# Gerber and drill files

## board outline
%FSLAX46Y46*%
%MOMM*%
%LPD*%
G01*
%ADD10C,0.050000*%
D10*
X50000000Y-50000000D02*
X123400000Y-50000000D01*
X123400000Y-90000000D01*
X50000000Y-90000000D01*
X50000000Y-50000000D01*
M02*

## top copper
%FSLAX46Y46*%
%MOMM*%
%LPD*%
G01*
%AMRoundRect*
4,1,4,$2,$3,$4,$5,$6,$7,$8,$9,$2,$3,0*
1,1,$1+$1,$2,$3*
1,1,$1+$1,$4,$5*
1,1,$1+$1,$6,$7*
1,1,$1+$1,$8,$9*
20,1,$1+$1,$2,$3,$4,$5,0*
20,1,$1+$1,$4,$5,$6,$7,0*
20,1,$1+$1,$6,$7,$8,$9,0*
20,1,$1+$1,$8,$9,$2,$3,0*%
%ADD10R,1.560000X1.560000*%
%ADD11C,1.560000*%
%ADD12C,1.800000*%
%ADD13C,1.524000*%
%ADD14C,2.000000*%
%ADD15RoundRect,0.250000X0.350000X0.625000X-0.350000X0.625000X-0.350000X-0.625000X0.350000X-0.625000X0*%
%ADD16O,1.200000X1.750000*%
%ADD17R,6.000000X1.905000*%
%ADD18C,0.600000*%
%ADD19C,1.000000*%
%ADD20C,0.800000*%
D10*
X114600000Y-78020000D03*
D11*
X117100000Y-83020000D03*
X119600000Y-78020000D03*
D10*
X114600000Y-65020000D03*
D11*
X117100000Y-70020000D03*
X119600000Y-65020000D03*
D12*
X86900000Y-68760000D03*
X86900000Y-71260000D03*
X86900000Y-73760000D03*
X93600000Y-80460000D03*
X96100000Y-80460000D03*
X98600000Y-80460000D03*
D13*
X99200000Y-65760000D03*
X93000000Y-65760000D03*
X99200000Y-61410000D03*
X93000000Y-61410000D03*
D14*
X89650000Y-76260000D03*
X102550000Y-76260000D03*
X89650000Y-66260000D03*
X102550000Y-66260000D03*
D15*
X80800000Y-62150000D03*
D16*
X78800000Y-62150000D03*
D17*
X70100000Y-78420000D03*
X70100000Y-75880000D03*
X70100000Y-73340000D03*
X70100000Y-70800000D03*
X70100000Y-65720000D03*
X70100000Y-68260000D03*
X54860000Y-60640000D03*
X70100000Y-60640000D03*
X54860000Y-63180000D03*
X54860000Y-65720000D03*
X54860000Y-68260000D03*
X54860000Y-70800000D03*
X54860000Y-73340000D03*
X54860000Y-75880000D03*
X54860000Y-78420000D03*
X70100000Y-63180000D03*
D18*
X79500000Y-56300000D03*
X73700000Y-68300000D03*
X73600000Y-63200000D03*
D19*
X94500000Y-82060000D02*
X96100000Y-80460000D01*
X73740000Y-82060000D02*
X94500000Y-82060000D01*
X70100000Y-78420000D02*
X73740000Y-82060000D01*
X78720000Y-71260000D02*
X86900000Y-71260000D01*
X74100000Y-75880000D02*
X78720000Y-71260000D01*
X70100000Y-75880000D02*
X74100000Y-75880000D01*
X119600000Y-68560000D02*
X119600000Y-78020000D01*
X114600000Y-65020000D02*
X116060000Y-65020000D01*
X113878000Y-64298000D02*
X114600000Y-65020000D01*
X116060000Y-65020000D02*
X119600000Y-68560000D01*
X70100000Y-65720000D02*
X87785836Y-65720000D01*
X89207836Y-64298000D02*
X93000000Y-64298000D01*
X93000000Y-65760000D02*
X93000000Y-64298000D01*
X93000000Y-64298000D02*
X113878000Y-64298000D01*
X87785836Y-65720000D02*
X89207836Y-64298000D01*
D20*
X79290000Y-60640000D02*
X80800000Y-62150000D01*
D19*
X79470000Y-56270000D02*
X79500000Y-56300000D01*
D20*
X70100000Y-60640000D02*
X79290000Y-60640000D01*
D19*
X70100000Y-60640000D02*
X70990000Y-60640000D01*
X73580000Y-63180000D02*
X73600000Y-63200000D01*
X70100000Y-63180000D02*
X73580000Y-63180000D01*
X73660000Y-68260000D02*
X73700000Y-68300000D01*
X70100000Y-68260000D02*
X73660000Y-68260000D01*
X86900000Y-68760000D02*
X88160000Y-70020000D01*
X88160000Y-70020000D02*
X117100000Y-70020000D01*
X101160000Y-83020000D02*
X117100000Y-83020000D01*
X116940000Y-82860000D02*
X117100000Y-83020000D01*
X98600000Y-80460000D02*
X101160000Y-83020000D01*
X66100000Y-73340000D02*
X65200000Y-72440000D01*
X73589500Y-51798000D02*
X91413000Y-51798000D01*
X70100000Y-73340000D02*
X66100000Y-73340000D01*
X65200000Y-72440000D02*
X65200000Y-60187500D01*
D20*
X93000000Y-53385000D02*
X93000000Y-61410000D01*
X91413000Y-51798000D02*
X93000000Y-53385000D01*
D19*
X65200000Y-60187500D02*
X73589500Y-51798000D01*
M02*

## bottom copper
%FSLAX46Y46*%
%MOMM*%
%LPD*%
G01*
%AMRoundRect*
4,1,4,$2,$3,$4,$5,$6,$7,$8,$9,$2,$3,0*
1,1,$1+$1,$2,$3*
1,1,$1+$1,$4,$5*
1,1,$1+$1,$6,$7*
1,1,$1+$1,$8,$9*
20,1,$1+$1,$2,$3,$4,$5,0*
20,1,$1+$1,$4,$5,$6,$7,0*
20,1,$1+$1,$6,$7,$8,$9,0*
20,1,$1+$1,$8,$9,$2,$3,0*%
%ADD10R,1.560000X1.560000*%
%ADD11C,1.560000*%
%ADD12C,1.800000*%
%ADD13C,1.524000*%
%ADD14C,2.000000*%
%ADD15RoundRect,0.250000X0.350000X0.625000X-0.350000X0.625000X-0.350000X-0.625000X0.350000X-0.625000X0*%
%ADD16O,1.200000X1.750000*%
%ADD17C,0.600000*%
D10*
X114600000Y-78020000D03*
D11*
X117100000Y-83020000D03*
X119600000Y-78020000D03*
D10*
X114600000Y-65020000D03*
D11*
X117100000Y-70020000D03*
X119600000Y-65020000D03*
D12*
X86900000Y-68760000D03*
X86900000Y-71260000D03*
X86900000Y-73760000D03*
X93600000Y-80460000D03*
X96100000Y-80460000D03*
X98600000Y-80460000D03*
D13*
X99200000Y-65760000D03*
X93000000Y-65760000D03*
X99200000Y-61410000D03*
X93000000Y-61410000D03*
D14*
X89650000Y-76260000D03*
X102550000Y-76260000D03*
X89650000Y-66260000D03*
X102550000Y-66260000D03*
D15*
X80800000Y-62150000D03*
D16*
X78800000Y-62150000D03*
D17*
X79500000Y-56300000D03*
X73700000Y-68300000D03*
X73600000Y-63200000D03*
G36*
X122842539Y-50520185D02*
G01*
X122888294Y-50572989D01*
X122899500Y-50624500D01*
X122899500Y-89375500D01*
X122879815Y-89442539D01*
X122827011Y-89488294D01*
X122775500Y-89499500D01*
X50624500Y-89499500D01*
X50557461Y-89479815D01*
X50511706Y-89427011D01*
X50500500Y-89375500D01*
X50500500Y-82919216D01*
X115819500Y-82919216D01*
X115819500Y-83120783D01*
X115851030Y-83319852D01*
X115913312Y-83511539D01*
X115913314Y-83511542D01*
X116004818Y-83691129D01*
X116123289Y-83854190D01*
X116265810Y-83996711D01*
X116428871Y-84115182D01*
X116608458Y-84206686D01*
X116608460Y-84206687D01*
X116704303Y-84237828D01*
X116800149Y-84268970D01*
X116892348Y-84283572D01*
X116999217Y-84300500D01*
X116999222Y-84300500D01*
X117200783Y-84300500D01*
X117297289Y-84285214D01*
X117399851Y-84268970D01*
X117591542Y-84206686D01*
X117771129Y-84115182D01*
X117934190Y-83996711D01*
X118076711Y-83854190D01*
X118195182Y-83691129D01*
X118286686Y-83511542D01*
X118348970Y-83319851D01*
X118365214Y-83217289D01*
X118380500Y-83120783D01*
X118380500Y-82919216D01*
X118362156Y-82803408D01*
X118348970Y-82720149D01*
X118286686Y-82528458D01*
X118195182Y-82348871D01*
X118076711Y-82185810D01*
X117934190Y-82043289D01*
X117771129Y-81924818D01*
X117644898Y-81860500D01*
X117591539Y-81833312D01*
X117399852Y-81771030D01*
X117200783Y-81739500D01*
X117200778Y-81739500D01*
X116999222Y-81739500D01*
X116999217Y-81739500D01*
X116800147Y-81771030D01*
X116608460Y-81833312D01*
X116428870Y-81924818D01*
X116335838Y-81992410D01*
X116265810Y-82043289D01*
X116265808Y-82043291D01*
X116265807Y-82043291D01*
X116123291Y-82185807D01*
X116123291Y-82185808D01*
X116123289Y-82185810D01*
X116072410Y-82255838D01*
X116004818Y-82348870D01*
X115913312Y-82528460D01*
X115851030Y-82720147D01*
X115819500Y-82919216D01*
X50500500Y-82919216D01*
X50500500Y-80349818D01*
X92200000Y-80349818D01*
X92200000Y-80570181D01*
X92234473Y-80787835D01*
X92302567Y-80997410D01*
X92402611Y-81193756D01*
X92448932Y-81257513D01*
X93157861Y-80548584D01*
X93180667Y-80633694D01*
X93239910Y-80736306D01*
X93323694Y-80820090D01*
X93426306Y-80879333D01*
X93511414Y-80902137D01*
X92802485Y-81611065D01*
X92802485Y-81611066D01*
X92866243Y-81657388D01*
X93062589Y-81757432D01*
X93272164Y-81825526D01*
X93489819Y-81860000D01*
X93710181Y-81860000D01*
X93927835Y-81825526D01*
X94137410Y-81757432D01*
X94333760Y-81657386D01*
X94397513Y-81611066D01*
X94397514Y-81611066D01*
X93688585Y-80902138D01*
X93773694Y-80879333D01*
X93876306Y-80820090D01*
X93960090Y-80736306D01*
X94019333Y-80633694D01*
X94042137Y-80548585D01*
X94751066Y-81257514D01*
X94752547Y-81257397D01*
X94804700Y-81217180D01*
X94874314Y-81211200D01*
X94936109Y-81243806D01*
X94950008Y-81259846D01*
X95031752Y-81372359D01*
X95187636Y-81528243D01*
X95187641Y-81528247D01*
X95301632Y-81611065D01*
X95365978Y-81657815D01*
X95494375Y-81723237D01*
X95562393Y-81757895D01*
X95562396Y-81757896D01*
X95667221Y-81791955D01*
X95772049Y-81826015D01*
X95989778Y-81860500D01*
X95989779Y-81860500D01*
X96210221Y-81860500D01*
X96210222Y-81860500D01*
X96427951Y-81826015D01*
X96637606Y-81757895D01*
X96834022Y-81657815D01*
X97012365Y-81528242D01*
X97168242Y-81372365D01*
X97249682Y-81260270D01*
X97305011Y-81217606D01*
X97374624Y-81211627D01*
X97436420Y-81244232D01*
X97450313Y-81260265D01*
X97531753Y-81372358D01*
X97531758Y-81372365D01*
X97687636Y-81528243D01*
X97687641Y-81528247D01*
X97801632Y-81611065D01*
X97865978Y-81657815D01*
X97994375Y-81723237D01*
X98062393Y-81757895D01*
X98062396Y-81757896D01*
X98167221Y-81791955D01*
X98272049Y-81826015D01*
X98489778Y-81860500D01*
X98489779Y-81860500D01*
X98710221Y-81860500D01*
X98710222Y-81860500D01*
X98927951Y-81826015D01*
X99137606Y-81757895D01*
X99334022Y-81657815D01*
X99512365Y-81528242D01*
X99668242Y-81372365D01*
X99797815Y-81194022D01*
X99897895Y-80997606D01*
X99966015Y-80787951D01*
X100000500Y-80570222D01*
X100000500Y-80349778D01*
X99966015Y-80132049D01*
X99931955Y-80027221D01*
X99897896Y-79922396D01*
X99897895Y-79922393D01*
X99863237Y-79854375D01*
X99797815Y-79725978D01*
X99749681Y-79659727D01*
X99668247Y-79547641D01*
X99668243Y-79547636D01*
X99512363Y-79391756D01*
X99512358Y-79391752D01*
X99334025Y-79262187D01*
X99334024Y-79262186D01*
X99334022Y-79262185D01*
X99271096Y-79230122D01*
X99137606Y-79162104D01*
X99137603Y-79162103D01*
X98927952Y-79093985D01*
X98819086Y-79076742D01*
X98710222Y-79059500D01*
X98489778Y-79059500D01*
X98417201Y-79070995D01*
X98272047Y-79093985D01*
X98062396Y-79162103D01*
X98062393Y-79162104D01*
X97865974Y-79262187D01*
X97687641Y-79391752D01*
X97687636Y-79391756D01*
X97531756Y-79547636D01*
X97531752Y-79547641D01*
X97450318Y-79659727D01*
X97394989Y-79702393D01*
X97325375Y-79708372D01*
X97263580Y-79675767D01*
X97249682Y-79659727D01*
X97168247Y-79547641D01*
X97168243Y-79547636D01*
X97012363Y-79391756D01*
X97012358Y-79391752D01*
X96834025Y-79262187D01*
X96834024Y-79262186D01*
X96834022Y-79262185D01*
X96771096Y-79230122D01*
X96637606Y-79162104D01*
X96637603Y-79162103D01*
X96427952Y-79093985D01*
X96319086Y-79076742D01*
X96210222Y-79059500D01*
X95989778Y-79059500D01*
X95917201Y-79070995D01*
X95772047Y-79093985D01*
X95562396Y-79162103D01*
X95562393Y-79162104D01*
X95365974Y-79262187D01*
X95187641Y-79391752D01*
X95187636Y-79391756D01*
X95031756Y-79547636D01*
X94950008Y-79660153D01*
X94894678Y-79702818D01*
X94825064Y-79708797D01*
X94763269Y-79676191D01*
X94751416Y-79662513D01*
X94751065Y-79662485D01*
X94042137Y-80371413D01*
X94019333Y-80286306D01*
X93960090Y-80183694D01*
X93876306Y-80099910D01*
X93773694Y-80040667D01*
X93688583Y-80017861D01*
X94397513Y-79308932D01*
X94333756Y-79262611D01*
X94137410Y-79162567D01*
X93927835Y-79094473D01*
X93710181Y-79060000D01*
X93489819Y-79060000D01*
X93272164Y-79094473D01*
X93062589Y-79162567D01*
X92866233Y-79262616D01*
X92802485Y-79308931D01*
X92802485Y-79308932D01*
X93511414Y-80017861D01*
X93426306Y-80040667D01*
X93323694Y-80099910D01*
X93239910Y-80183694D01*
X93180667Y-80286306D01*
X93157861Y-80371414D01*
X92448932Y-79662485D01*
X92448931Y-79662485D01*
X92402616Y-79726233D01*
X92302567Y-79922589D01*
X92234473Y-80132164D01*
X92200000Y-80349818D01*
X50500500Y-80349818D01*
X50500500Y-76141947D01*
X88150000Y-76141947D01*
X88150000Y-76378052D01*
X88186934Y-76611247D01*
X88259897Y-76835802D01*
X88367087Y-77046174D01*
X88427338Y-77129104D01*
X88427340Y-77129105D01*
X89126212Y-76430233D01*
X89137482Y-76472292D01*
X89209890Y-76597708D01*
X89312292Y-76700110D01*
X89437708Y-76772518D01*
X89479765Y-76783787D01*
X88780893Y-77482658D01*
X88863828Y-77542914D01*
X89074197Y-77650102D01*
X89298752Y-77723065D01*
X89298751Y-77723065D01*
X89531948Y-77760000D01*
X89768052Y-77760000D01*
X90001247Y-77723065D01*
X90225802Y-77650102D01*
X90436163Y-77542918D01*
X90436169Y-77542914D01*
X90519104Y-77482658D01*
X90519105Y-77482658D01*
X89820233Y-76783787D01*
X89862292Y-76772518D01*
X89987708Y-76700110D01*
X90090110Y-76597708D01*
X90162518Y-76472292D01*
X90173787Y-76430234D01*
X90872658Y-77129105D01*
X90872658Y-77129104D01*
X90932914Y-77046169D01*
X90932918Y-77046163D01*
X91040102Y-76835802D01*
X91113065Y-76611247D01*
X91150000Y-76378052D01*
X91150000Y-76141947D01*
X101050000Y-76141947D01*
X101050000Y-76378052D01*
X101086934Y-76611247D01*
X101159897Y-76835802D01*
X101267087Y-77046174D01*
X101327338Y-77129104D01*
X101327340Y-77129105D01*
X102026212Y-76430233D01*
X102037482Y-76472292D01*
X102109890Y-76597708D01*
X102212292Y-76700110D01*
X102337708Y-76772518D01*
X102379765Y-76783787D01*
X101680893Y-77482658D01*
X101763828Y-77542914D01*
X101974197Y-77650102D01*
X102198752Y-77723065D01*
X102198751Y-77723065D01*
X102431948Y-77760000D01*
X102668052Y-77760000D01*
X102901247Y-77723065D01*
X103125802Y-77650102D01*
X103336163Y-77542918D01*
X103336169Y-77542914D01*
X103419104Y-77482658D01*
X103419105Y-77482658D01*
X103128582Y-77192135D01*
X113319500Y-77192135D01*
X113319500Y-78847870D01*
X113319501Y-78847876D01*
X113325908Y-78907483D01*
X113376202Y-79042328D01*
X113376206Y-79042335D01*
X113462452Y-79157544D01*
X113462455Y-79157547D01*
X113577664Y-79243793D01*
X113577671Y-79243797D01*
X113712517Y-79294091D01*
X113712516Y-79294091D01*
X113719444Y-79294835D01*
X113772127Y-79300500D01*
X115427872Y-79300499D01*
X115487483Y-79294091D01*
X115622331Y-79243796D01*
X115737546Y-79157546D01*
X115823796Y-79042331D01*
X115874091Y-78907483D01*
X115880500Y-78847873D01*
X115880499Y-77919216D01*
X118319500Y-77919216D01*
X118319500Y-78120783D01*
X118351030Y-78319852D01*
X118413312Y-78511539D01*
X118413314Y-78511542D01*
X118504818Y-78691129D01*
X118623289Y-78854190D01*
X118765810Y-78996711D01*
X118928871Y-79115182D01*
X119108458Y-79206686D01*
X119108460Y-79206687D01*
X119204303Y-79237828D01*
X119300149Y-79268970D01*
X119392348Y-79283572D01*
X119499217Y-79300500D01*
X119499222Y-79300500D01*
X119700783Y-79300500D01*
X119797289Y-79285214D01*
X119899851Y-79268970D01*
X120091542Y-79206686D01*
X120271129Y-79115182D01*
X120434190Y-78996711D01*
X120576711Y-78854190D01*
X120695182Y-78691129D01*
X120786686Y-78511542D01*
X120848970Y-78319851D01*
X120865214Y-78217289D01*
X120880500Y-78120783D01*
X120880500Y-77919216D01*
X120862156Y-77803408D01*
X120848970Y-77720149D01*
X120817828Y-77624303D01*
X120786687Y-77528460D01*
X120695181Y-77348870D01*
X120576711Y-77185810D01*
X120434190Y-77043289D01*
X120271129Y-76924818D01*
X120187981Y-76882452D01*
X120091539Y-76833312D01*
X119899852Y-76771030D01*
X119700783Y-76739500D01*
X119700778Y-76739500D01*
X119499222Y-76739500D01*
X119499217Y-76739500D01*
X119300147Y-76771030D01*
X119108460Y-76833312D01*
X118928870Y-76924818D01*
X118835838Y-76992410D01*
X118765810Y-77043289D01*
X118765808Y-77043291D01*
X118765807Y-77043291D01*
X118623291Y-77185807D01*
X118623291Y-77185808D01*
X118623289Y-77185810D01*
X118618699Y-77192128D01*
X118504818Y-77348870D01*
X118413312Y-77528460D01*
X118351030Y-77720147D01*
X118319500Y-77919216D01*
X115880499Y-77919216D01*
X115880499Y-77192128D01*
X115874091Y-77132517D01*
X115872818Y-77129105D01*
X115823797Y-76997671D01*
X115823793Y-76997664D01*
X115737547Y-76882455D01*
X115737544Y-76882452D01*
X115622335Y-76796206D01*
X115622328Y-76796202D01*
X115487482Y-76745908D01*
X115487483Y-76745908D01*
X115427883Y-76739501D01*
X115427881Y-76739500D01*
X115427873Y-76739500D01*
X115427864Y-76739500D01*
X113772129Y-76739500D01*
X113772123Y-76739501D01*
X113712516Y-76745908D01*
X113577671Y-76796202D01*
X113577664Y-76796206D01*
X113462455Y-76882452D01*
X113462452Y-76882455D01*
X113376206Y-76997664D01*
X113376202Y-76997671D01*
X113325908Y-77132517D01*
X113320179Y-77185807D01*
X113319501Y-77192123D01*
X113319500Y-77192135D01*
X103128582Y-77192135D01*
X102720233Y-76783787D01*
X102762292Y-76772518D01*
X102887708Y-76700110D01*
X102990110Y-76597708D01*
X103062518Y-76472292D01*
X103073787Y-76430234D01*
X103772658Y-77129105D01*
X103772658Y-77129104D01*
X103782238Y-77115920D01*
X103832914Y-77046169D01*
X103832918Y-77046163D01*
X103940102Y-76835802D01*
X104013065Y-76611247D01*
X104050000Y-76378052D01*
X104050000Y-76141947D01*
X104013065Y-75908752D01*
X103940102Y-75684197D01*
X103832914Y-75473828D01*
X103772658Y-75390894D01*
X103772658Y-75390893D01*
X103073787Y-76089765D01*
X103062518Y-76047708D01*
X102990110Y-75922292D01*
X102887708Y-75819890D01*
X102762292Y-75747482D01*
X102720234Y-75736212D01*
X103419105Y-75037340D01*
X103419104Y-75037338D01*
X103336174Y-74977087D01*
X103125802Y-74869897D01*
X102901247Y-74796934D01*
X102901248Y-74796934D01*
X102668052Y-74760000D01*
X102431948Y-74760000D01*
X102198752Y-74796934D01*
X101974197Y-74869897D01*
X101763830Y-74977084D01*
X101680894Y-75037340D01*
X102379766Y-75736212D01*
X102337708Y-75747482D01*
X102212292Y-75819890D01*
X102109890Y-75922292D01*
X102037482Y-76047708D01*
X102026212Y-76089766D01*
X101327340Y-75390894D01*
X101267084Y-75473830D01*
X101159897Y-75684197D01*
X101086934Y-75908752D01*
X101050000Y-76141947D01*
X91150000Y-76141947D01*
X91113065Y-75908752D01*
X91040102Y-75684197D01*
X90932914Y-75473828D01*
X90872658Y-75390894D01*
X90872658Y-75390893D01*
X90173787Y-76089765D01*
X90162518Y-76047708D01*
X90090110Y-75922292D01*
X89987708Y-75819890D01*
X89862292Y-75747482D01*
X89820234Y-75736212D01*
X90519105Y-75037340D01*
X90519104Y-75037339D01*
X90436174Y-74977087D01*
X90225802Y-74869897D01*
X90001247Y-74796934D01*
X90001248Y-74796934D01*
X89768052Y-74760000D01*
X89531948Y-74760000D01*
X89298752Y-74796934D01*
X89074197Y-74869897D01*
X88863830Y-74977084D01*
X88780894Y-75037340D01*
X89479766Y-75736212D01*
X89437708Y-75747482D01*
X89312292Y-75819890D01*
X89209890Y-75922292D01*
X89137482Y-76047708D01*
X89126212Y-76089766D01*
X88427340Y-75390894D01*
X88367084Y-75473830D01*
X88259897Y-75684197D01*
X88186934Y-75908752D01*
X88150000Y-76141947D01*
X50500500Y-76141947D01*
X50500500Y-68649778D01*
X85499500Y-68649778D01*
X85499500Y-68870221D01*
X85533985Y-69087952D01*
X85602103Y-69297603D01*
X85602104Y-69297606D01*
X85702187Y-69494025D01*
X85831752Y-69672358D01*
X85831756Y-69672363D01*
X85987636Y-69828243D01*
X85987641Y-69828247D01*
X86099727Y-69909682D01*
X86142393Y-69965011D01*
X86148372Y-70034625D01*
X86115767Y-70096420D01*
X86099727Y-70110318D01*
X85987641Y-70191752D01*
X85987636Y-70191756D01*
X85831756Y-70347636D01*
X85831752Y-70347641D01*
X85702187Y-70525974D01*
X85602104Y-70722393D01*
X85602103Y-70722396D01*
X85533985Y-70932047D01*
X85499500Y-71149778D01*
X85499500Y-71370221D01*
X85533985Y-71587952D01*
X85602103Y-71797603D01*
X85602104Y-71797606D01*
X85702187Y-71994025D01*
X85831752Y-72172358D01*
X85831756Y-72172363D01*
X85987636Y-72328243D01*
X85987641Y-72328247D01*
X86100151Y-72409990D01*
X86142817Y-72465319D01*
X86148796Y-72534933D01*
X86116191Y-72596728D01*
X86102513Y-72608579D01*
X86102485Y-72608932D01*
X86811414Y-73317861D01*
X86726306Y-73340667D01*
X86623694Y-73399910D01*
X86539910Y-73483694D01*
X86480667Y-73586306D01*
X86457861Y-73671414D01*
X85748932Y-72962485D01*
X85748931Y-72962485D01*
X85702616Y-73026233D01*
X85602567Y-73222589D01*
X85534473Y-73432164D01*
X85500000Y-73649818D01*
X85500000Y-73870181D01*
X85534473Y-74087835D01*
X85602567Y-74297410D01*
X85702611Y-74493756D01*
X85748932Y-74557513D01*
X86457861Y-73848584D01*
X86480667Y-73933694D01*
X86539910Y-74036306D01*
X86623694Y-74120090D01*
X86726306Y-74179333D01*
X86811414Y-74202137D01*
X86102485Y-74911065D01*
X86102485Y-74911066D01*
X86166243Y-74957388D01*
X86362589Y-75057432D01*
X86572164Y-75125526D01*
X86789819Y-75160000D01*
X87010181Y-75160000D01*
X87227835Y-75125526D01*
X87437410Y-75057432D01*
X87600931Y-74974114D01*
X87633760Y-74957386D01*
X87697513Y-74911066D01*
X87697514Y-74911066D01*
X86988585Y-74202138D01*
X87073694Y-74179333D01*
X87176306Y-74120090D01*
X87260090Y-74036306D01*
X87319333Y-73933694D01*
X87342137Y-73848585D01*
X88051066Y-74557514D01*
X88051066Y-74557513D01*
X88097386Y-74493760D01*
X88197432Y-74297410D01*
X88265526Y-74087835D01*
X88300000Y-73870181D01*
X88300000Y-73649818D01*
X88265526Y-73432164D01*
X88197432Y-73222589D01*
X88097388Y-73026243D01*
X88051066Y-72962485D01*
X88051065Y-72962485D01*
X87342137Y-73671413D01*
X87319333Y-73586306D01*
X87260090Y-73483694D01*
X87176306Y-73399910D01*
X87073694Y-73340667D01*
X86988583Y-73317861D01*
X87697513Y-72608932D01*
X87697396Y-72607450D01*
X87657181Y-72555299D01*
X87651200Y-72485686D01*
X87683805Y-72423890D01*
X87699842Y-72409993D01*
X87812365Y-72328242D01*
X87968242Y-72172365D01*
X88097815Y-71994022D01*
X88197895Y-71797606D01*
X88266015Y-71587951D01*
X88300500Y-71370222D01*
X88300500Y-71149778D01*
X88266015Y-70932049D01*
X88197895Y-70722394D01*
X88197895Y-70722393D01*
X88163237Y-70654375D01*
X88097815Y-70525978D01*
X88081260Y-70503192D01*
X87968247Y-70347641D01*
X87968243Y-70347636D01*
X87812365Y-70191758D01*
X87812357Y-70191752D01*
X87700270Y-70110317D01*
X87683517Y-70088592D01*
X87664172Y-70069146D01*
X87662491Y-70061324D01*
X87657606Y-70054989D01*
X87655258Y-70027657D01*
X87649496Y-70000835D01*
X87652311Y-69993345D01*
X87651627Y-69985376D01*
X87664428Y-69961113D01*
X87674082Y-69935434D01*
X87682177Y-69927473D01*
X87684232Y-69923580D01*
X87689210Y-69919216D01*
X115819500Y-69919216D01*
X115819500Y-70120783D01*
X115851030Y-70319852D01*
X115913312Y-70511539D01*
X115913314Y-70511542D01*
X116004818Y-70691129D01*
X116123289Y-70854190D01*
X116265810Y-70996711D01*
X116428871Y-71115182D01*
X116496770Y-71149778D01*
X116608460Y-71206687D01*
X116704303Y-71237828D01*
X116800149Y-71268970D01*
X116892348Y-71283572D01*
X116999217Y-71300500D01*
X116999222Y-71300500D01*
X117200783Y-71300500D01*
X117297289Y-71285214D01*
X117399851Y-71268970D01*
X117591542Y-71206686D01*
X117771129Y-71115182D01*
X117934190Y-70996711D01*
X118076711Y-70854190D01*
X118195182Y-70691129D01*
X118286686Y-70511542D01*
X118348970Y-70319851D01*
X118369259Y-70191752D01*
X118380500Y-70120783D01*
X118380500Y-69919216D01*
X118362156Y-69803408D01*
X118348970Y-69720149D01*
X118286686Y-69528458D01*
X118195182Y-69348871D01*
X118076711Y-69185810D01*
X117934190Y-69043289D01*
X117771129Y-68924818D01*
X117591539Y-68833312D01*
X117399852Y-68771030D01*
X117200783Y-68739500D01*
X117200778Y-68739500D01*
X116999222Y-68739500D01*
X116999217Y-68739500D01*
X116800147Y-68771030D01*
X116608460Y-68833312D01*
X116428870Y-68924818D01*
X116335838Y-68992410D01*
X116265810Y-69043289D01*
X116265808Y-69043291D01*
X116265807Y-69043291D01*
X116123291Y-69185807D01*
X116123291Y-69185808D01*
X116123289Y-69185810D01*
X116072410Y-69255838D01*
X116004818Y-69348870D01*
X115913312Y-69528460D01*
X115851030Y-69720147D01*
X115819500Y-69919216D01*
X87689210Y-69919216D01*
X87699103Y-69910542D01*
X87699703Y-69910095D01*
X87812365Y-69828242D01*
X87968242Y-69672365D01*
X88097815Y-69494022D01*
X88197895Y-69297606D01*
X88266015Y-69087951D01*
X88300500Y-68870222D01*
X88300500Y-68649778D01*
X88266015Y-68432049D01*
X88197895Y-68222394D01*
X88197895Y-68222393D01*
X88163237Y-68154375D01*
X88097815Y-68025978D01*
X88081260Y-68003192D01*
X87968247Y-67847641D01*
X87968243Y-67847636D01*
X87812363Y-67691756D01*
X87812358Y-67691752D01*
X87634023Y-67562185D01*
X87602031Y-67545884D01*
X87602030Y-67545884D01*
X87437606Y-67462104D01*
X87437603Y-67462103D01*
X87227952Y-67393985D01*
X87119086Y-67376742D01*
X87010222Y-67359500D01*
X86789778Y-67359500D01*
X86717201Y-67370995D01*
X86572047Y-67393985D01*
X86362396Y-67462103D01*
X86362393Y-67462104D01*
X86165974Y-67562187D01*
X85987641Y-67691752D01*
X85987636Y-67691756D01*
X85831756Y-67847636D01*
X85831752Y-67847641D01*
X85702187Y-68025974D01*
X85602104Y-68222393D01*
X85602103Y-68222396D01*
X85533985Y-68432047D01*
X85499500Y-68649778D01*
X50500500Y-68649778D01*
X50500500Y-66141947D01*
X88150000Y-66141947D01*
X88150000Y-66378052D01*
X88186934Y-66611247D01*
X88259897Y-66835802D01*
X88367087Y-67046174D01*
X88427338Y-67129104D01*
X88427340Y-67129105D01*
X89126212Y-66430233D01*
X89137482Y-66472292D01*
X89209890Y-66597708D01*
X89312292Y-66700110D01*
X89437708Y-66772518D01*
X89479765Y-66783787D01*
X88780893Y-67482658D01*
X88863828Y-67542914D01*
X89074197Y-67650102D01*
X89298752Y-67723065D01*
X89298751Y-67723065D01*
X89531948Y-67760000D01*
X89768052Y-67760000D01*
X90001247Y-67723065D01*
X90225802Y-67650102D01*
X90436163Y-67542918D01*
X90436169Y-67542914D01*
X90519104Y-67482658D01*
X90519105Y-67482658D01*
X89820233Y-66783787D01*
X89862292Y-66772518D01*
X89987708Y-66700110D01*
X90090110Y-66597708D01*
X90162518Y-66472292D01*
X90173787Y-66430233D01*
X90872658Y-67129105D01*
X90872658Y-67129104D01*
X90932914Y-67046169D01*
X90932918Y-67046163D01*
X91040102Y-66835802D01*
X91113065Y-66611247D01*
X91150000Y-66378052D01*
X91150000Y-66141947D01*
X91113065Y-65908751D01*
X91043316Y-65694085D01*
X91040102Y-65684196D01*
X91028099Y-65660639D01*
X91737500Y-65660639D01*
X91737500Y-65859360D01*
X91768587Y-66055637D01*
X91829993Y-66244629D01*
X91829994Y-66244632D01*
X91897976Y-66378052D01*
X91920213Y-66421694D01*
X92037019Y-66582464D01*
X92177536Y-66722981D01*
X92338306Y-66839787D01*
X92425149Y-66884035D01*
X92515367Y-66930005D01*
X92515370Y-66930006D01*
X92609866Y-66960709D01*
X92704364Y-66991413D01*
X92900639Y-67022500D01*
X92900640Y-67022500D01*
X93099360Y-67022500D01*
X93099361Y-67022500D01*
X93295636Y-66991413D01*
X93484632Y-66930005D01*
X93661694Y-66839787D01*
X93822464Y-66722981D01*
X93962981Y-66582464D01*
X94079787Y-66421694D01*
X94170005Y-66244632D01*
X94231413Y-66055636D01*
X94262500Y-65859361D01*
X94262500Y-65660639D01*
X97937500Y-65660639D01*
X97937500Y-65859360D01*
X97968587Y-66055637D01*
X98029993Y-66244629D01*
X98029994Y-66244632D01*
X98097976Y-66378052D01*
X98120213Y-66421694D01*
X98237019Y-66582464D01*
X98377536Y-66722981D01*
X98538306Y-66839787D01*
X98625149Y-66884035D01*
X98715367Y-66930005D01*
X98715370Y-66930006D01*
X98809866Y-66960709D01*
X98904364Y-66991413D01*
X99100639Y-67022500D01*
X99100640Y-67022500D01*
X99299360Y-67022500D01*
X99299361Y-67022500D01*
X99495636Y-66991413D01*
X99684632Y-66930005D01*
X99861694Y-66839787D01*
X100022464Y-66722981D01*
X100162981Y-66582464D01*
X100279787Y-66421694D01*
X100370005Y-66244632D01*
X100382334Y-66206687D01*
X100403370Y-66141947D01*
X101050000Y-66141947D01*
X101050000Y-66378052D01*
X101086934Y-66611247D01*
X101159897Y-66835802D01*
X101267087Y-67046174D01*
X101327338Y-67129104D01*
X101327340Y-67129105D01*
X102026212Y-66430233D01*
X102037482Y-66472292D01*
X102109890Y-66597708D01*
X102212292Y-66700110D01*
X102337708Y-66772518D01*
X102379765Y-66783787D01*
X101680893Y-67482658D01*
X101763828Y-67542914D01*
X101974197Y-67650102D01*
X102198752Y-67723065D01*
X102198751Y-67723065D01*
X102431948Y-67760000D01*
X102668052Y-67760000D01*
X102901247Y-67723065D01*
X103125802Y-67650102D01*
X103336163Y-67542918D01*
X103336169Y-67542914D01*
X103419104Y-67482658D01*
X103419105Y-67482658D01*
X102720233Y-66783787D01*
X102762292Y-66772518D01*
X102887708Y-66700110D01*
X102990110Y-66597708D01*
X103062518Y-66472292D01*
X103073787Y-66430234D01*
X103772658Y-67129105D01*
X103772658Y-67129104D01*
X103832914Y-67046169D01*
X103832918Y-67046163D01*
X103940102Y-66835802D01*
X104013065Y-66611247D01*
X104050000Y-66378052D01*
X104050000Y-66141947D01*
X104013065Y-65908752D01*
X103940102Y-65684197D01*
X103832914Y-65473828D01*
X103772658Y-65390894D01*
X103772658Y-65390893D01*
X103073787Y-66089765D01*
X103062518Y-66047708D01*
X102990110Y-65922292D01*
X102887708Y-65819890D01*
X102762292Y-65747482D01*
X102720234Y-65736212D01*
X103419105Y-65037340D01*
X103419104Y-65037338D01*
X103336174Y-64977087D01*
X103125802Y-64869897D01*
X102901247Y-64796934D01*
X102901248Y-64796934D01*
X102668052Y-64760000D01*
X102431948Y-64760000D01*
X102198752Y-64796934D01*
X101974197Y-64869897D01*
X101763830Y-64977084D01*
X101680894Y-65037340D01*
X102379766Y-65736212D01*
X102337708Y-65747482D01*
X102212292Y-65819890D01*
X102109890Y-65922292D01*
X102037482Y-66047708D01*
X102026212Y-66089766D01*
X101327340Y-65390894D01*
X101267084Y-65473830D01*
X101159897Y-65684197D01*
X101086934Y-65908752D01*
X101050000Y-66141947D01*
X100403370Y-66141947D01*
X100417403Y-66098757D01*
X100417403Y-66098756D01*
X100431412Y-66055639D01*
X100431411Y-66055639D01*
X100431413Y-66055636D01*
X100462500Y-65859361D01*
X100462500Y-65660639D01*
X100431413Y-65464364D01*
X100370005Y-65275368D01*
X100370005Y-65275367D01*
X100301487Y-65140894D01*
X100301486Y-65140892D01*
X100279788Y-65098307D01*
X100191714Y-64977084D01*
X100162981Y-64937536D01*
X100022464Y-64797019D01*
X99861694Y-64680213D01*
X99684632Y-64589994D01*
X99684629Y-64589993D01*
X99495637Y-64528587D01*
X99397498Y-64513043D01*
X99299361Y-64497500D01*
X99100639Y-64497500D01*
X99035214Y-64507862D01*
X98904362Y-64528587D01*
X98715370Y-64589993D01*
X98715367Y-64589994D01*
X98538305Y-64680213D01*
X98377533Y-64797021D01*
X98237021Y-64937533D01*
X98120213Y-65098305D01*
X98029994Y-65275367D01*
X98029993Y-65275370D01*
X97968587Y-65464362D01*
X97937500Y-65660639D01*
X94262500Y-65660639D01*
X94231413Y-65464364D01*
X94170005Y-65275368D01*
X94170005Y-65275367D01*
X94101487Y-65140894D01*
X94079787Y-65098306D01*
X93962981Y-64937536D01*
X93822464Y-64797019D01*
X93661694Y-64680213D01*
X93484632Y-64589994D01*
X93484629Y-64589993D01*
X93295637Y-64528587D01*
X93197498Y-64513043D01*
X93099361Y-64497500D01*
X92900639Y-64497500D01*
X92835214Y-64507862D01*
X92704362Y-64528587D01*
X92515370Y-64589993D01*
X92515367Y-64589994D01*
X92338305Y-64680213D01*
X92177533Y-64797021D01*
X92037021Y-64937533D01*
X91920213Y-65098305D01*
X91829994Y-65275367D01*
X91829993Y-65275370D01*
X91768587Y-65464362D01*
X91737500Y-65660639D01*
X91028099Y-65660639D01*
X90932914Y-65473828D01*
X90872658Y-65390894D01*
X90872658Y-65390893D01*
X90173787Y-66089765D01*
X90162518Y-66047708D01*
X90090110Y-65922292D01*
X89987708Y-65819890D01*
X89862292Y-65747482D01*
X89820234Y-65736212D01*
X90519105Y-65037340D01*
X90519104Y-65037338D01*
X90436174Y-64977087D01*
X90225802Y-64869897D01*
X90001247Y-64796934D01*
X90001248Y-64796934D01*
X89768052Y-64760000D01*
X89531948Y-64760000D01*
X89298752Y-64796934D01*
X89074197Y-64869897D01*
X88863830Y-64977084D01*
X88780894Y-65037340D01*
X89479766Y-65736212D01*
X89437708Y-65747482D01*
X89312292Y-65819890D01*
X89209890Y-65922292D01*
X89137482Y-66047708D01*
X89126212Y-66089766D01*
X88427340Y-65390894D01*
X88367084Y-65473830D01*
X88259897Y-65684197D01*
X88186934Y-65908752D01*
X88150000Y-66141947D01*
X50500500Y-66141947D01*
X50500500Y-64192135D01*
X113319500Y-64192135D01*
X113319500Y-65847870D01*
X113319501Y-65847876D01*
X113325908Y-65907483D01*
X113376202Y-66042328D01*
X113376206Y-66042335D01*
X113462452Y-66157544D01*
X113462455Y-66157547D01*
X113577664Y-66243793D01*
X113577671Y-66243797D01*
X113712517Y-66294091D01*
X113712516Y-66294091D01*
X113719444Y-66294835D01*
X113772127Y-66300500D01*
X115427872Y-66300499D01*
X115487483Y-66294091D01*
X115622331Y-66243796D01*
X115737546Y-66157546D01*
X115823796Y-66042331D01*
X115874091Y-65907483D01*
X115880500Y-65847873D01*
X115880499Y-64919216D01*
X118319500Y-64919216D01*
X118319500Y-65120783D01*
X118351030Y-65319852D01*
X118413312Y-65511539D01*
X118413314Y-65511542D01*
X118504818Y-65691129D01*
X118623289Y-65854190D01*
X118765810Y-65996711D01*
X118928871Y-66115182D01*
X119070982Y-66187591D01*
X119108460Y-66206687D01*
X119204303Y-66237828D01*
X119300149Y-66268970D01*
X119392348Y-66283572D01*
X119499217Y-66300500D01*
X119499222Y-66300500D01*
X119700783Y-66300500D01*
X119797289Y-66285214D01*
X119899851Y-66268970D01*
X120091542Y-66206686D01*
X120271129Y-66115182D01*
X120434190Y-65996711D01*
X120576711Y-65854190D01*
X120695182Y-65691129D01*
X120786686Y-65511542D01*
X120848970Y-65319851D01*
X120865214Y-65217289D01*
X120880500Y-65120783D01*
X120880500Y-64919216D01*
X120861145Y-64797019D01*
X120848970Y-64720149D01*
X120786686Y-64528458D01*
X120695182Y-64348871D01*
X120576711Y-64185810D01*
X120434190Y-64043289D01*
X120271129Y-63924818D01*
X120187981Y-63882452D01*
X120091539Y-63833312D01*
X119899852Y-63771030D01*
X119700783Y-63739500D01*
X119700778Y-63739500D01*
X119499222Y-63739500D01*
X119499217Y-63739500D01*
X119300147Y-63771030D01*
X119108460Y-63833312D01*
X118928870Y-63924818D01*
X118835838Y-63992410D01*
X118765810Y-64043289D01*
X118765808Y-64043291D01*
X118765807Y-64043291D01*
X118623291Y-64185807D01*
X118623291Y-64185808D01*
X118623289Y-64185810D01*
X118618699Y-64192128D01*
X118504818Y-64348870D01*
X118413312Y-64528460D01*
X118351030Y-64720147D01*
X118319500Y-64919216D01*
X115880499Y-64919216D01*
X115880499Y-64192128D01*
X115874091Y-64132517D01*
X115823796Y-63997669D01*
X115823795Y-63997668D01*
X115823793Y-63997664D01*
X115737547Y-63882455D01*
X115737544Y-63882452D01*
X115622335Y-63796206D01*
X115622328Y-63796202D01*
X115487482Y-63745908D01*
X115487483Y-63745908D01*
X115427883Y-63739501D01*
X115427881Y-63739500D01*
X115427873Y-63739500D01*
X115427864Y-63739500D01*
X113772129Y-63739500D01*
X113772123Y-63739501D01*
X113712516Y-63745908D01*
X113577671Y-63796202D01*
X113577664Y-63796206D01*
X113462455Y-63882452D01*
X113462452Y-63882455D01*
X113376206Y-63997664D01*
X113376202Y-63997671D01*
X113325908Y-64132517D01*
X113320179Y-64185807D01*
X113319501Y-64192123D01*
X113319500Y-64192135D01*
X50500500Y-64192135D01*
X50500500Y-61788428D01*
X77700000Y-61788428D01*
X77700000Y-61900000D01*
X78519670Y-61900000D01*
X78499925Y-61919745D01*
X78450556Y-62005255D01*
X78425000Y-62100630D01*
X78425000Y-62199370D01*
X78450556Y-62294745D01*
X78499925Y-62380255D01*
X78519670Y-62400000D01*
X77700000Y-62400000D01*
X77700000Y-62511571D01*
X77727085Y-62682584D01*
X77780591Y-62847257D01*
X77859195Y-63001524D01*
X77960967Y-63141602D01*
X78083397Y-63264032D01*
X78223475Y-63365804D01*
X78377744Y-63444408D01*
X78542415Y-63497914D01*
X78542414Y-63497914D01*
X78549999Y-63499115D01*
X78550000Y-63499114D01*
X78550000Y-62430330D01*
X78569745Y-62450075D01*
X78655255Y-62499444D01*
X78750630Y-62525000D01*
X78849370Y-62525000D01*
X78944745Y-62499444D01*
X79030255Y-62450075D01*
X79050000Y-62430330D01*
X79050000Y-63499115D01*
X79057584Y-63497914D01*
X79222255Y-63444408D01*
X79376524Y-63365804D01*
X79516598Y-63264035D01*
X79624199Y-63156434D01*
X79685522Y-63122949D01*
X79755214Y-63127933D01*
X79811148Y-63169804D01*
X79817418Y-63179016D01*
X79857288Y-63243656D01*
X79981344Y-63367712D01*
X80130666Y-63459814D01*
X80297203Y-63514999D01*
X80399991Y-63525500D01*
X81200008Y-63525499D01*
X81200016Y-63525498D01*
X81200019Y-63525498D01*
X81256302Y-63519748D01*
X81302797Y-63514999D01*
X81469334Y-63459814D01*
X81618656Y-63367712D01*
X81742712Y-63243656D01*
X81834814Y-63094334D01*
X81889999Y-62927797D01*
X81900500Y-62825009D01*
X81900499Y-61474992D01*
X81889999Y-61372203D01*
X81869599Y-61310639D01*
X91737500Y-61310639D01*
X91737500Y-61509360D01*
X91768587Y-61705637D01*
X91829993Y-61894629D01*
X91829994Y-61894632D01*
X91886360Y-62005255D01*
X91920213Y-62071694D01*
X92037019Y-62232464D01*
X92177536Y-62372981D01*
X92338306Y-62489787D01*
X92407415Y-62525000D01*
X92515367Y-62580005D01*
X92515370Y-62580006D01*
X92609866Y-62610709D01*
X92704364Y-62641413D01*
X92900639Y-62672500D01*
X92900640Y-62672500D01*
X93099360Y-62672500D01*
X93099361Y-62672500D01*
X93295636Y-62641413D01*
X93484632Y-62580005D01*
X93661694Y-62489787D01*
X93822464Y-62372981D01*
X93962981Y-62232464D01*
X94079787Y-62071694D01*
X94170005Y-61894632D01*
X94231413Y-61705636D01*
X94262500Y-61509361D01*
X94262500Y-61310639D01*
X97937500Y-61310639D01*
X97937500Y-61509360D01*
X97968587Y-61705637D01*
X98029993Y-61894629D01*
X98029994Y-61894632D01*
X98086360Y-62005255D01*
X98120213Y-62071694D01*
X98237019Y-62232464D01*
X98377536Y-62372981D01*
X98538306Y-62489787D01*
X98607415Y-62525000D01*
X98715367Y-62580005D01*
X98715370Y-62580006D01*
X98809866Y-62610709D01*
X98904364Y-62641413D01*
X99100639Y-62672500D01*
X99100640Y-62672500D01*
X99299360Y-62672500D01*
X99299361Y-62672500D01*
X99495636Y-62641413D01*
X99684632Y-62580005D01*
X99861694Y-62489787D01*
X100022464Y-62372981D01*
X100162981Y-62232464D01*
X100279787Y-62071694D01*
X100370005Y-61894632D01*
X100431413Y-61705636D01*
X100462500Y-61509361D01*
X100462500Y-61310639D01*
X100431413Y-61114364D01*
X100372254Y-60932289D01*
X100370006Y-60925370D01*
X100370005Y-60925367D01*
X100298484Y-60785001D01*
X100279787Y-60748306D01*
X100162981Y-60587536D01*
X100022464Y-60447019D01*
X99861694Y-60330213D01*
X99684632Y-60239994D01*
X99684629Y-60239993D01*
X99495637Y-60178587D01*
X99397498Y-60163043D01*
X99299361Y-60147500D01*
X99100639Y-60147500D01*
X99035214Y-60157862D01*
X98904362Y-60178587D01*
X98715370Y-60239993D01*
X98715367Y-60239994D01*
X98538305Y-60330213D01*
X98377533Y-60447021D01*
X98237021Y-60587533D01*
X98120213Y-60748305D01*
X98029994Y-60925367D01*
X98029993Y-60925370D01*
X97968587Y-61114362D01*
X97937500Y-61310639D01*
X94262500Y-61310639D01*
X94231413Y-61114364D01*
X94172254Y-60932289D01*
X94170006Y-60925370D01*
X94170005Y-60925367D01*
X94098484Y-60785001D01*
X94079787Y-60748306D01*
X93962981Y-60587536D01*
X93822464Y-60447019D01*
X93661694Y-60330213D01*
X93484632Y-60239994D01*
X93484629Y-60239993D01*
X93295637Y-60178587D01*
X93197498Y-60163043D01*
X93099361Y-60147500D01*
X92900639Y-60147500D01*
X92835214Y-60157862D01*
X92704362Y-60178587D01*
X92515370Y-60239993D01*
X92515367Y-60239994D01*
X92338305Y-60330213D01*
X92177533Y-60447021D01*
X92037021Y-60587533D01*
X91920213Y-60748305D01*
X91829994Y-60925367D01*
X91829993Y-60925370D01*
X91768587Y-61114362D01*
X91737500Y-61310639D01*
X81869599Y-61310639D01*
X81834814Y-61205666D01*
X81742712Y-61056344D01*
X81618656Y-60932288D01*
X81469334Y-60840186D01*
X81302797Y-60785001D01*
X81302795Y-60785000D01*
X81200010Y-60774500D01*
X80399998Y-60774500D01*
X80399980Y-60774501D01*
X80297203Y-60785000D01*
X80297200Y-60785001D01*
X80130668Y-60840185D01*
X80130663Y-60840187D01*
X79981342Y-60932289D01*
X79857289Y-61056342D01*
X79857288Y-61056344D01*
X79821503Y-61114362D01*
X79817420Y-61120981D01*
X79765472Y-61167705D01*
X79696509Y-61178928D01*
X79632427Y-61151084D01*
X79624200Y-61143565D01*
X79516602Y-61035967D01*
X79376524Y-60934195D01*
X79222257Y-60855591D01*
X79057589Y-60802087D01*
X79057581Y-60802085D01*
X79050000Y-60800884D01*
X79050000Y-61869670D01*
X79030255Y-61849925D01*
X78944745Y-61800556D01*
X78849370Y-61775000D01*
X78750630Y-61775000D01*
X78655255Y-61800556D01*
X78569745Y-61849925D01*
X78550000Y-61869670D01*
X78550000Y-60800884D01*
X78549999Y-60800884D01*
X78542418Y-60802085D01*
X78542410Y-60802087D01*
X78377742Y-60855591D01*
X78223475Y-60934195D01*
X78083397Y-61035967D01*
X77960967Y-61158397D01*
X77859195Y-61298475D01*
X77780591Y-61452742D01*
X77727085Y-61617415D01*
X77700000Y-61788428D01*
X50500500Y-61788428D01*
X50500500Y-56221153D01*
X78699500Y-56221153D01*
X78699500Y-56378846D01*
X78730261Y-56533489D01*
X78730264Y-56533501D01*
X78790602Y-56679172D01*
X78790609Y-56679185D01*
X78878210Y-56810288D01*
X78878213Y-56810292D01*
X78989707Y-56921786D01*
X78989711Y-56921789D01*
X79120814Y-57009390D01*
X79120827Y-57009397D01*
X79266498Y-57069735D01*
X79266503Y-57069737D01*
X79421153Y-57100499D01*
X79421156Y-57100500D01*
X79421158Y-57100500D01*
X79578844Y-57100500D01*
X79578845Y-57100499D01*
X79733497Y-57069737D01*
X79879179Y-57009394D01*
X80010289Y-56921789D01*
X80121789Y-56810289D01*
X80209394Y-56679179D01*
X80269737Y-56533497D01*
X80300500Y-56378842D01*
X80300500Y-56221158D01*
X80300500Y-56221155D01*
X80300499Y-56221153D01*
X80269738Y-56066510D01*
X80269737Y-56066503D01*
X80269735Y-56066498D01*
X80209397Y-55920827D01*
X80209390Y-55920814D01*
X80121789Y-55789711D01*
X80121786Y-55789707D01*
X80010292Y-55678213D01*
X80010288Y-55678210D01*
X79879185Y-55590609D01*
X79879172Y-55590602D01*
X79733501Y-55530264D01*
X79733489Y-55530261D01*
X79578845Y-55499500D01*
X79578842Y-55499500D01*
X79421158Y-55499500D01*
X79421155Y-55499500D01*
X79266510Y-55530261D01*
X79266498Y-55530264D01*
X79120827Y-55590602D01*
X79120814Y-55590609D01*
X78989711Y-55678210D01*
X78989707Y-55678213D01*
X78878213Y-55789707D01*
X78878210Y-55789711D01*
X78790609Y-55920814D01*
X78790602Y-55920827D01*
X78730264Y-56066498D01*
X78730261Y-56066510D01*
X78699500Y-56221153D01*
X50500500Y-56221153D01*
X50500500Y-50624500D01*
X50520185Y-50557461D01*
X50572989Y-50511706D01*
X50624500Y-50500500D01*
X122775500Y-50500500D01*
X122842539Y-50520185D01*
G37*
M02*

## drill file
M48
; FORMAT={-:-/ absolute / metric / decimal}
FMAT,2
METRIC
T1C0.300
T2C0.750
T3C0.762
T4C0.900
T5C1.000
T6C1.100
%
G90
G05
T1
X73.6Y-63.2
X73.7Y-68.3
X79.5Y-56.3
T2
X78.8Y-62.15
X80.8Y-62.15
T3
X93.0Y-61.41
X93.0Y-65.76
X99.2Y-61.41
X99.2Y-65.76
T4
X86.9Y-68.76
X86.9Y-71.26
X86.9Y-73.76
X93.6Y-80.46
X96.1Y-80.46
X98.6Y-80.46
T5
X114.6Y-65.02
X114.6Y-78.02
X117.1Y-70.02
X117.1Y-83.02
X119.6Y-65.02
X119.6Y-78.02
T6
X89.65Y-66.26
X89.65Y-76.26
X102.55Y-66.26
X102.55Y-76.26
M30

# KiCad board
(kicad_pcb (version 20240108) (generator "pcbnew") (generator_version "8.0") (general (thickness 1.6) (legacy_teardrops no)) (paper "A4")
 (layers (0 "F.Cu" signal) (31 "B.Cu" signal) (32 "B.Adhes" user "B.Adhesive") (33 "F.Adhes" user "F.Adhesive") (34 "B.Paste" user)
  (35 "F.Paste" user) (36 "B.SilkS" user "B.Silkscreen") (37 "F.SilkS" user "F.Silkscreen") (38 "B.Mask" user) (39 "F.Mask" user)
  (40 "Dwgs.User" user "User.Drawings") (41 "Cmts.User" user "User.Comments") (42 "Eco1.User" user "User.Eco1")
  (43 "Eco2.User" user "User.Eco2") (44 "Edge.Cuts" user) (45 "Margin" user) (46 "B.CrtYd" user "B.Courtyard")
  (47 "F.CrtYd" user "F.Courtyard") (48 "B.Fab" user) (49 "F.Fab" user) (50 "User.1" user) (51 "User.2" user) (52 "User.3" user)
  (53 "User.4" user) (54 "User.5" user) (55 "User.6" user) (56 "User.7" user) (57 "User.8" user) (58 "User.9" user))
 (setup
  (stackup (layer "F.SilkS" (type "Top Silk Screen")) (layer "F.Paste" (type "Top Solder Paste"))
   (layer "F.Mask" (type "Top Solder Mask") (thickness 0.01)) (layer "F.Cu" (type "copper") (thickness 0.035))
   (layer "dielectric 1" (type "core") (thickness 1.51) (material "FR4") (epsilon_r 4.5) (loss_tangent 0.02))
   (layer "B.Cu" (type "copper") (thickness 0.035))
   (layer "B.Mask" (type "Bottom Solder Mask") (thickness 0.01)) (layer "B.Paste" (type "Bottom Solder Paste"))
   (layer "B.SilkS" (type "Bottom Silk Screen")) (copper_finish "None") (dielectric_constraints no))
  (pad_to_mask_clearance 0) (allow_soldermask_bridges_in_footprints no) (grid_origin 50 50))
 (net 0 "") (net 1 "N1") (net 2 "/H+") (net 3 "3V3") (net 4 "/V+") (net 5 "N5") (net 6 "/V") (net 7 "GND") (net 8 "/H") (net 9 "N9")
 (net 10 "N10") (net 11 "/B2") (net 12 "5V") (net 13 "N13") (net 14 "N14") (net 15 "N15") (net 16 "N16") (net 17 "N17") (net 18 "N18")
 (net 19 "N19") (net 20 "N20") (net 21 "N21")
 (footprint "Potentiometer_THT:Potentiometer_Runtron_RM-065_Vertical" (layer "F.Cu") (at 114.6 78.02)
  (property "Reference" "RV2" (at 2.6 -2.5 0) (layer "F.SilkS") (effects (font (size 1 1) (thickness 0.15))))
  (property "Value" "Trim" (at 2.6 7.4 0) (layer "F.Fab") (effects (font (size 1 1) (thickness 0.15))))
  (pad "1" thru_hole rect (at 0 0) (size 1.56 1.56) (drill 1) (layers "*.Cu" "*.Mask") (remove_unused_layers no) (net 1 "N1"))
  (pad "2" thru_hole circle (at 2.5 5) (size 1.56 1.56) (drill 1) (layers "*.Cu" "*.Mask") (remove_unused_layers no) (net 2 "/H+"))
  (pad "3" thru_hole circle (at 5 0) (size 1.56 1.56) (drill 1) (layers "*.Cu" "*.Mask") (remove_unused_layers no) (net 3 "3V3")))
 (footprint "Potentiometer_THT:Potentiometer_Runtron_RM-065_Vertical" (layer "F.Cu") (at 114.6 65.02)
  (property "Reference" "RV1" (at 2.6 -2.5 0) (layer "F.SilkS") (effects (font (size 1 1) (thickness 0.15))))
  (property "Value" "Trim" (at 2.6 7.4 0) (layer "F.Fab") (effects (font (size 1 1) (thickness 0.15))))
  (pad "1" thru_hole rect (at 0 0) (size 1.56 1.56) (drill 1) (layers "*.Cu" "*.Mask") (remove_unused_layers no) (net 3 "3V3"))
  (pad "2" thru_hole circle (at 2.5 5) (size 1.56 1.56) (drill 1) (layers "*.Cu" "*.Mask") (remove_unused_layers no) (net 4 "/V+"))
  (pad "3" thru_hole circle (at 5 0) (size 1.56 1.56) (drill 1) (layers "*.Cu" "*.Mask") (remove_unused_layers no) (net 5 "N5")))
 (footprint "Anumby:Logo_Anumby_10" (layer "F.Cu") (at 112.2 55.4)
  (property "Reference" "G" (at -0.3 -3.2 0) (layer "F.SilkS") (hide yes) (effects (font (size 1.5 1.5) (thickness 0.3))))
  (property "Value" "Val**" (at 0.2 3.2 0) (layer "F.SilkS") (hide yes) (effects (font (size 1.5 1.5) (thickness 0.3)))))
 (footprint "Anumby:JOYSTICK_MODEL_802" (layer "F.Cu") (at 96.1 71.26 -90)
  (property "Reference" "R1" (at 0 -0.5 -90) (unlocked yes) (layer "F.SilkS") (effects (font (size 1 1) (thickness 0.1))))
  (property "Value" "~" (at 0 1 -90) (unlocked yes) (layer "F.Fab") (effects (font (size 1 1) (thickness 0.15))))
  (pad "1" thru_hole circle (at -2.5 9.2 270) (size 1.8 1.8) (drill 0.9) (layers "*.Cu" "*.Mask") (remove_unused_layers no) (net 4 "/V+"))
  (pad "2" thru_hole circle (at 0 9.2 270) (size 1.8 1.8) (drill 0.9) (layers "*.Cu" "*.Mask") (remove_unused_layers no) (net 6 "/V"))
  (pad "3" thru_hole circle (at 2.5 9.2 270) (size 1.8 1.8) (drill 0.9) (layers "*.Cu" "*.Mask") (remove_unused_layers no) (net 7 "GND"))
  (pad "4" thru_hole circle (at 9.2 2.5 270) (size 1.8 1.8) (drill 0.9) (layers "*.Cu" "*.Mask") (remove_unused_layers no) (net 7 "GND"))
  (pad "5" thru_hole circle (at 9.2 0 270) (size 1.8 1.8) (drill 0.9) (layers "*.Cu" "*.Mask") (remove_unused_layers no) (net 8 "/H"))
  (pad "6" thru_hole circle (at 9.2 -2.5 270) (size 1.8 1.8) (drill 0.9) (layers "*.Cu" "*.Mask") (remove_unused_layers no) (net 2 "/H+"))
  (pad "7" thru_hole circle (at -5.5 -3.1 270) (size 1.524 1.524) (drill 0.762) (layers "*.Cu" "*.Mask") (remove_unused_layers no)
   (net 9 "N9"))
  (pad "8" thru_hole circle (at -5.5 3.1 270) (size 1.524 1.524) (drill 0.762) (layers "*.Cu" "*.Mask") (remove_unused_layers no)
   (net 3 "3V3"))
  (pad "9" thru_hole circle (at -9.85 -3.1 270) (size 1.524 1.524) (drill 0.762) (layers "*.Cu" "*.Mask") (remove_unused_layers no)
   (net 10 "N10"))
  (pad "10" thru_hole circle (at -9.85 3.1 270) (size 1.524 1.524) (drill 0.762) (layers "*.Cu" "*.Mask") (remove_unused_layers no)
   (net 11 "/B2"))
  (pad "11" thru_hole circle (at 5 6.45 270) (size 2 2) (drill 1.1) (layers "*.Cu" "*.Mask") (remove_unused_layers no) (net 7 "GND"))
  (pad "12" thru_hole circle (at 5 -6.45 270) (size 2 2) (drill 1.1) (layers "*.Cu" "*.Mask") (remove_unused_layers no) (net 7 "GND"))
  (pad "13" thru_hole circle (at -5 6.45 270) (size 2 2) (drill 1.1) (layers "*.Cu" "*.Mask") (remove_unused_layers no) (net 7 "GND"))
  (pad "14" thru_hole circle (at -5 -6.45 270) (size 2 2) (drill 1.1) (layers "*.Cu" "*.Mask") (remove_unused_layers no) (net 7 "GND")))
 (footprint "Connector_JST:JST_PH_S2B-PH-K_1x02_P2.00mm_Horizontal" (layer "F.Cu") (at 80.8 62.15 180)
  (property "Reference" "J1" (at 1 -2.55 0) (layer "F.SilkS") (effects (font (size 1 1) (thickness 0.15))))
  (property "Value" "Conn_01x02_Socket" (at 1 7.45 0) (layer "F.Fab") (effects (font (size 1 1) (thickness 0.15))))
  (pad "1" thru_hole roundrect (at 0 0 180) (size 1.2 1.75) (drill 0.75) (layers "*.Cu" "*.Mask") (remove_unused_layers no)
   (roundrect_rratio 0.208333) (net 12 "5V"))
  (pad "2" thru_hole oval (at 2 0 180) (size 1.2 1.75) (drill 0.75) (layers "*.Cu" "*.Mask") (remove_unused_layers no) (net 7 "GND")))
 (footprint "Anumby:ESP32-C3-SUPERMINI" (layer "F.Cu") (at 62.48 70.54)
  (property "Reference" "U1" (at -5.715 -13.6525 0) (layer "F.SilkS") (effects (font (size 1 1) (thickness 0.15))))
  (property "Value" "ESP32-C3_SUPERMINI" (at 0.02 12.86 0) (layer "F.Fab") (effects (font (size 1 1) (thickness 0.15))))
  (pad "0" smd rect (at 7.62 7.88) (size 6 1.905) (layers "F.Cu" "F.Paste" "F.Mask") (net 8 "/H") (solder_mask_margin 0.102))
  (pad "1" smd rect (at 7.62 5.34) (size 6 1.905) (layers "F.Cu" "F.Paste" "F.Mask") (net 6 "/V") (solder_mask_margin 0.102))
  (pad "2" smd rect (at 7.62 2.8) (size 6 1.905) (layers "F.Cu" "F.Paste" "F.Mask") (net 11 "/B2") (solder_mask_margin 0.102))
  (pad "3" smd rect (at 7.62 0.26) (size 6 1.905) (layers "F.Cu" "F.Paste" "F.Mask") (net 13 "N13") (solder_mask_margin 0.102))
  (pad "3.3" smd rect (at 7.62 -4.82) (size 6 1.905) (layers "F.Cu" "F.Paste" "F.Mask") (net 3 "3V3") (solder_mask_margin 0.102))
  (pad "4" smd rect (at 7.62 -2.28) (size 6 1.905) (layers "F.Cu" "F.Paste" "F.Mask") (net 7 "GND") (solder_mask_margin 0.102))
  (pad "5" smd rect (at -7.62 -9.9) (size 6 1.905) (layers "F.Cu" "F.Paste" "F.Mask") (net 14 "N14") (solder_mask_margin 0.102))
  (pad "5V" smd rect (at 7.62 -9.9) (size 6 1.905) (layers "F.Cu" "F.Paste" "F.Mask") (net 12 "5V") (solder_mask_margin 0.102))
  (pad "6" smd rect (at -7.62 -7.36) (size 6 1.905) (layers "F.Cu" "F.Paste" "F.Mask") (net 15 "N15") (solder_mask_margin 0.102))
  (pad "7" smd rect (at -7.62 -4.82) (size 6 1.905) (layers "F.Cu" "F.Paste" "F.Mask") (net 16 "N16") (solder_mask_margin 0.102))
  (pad "8" smd rect (at -7.62 -2.28) (size 6 1.905) (layers "F.Cu" "F.Paste" "F.Mask") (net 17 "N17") (solder_mask_margin 0.102))
  (pad "9" smd rect (at -7.62 0.26) (size 6 1.905) (layers "F.Cu" "F.Paste" "F.Mask") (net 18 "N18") (solder_mask_margin 0.102))
  (pad "10" smd rect (at -7.62 2.8) (size 6 1.905) (layers "F.Cu" "F.Paste" "F.Mask") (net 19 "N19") (solder_mask_margin 0.102))
  (pad "20" smd rect (at -7.62 5.34) (size 6 1.905) (layers "F.Cu" "F.Paste" "F.Mask") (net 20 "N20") (solder_mask_margin 0.102))
  (pad "21" smd rect (at -7.62 7.88) (size 6 1.905) (layers "F.Cu" "F.Paste" "F.Mask") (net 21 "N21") (solder_mask_margin 0.102))
  (pad "G" smd rect (at 7.62 -7.36) (size 6 1.905) (layers "F.Cu" "F.Paste" "F.Mask") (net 7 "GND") (solder_mask_margin 0.102)))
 (gr_rect (start 50 50) (end 123.4 90) (stroke (width 0.05) (type default)) (fill none) (layer "Edge.Cuts"))
 (segment (start 94.5 82.06) (end 96.1 80.46) (width 1) (layer "F.Cu") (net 8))
 (segment (start 73.74 82.06) (end 94.5 82.06) (width 1) (layer "F.Cu") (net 8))
 (segment (start 70.1 78.42) (end 73.74 82.06) (width 1) (layer "F.Cu") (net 8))
 (segment (start 78.72 71.26) (end 86.9 71.26) (width 1) (layer "F.Cu") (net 6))
 (segment (start 74.1 75.88) (end 78.72 71.26) (width 1) (layer "F.Cu") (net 6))
 (segment (start 70.1 75.88) (end 74.1 75.88) (width 1) (layer "F.Cu") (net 6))
 (segment (start 119.6 68.56) (end 119.6 78.02) (width 1) (layer "F.Cu") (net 3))
 (segment (start 114.6 65.02) (end 116.06 65.02) (width 1) (layer "F.Cu") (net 3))
 (segment (start 113.878 64.298) (end 114.6 65.02) (width 1) (layer "F.Cu") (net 3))
 (segment (start 116.06 65.02) (end 119.6 68.56) (width 1) (layer "F.Cu") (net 3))
 (segment (start 70.1 65.72) (end 87.785836 65.72) (width 1) (layer "F.Cu") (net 3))
 (segment (start 89.207836 64.298) (end 93 64.298) (width 1) (layer "F.Cu") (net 3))
 (segment (start 93 65.76) (end 93 64.298) (width 1) (layer "F.Cu") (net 3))
 (segment (start 93 64.298) (end 113.878 64.298) (width 1) (layer "F.Cu") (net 3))
 (segment (start 87.785836 65.72) (end 89.207836 64.298) (width 1) (layer "F.Cu") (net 3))
 (segment (start 79.29 60.64) (end 80.8 62.15) (width 0.8) (layer "F.Cu") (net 12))
 (segment (start 79.47 56.27) (end 79.5 56.3) (width 1) (layer "F.Cu") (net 12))
 (segment (start 70.1 60.64) (end 79.29 60.64) (width 0.8) (layer "F.Cu") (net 12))
 (segment (start 70.1 60.64) (end 70.99 60.64) (width 1) (layer "F.Cu") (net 12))
 (via (at 79.5 56.3) (size 0.6) (drill 0.3) (layers "F.Cu" "B.Cu") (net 12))
 (segment (start 73.58 63.18) (end 73.6 63.2) (width 1) (layer "F.Cu") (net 7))
 (segment (start 70.1 63.18) (end 73.58 63.18) (width 1) (layer "F.Cu") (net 7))
 (segment (start 73.66 68.26) (end 73.7 68.3) (width 1) (layer "F.Cu") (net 7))
 (segment (start 70.1 68.26) (end 73.66 68.26) (width 1) (layer "F.Cu") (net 7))
 (via (at 73.7 68.3) (size 0.6) (drill 0.3) (layers "F.Cu" "B.Cu") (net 7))
 (via (at 73.6 63.2) (size 0.6) (drill 0.3) (layers "F.Cu" "B.Cu") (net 7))
 (segment (start 86.9 68.76) (end 88.16 70.02) (width 1) (layer "F.Cu") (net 4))
 (segment (start 88.16 70.02) (end 117.1 70.02) (width 1) (layer "F.Cu") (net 4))
 (segment (start 101.16 83.02) (end 117.1 83.02) (width 1) (layer "F.Cu") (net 2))
 (segment (start 116.94 82.86) (end 117.1 83.02) (width 1) (layer "F.Cu") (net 2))
 (segment (start 98.6 80.46) (end 101.16 83.02) (width 1) (layer "F.Cu") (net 2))
 (segment (start 66.1 73.34) (end 65.2 72.44) (width 1) (layer "F.Cu") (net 11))
 (segment (start 73.5895 51.798) (end 91.413 51.798) (width 1) (layer "F.Cu") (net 11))
 (segment (start 70.1 73.34) (end 66.1 73.34) (width 1) (layer "F.Cu") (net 11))
 (segment (start 65.2 72.44) (end 65.2 60.1875) (width 1) (layer "F.Cu") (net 11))
 (segment (start 93 53.385) (end 93 61.41) (width 0.8) (layer "F.Cu") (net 11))
 (segment (start 91.413 51.798) (end 93 53.385) (width 0.8) (layer "F.Cu") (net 11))
 (segment (start 65.2 60.1875) (end 73.5895 51.798) (width 1) (layer "F.Cu") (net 11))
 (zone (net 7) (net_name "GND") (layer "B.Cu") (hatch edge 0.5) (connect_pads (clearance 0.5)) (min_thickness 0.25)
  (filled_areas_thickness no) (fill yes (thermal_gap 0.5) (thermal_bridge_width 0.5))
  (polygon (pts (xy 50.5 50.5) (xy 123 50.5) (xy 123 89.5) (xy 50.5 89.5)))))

